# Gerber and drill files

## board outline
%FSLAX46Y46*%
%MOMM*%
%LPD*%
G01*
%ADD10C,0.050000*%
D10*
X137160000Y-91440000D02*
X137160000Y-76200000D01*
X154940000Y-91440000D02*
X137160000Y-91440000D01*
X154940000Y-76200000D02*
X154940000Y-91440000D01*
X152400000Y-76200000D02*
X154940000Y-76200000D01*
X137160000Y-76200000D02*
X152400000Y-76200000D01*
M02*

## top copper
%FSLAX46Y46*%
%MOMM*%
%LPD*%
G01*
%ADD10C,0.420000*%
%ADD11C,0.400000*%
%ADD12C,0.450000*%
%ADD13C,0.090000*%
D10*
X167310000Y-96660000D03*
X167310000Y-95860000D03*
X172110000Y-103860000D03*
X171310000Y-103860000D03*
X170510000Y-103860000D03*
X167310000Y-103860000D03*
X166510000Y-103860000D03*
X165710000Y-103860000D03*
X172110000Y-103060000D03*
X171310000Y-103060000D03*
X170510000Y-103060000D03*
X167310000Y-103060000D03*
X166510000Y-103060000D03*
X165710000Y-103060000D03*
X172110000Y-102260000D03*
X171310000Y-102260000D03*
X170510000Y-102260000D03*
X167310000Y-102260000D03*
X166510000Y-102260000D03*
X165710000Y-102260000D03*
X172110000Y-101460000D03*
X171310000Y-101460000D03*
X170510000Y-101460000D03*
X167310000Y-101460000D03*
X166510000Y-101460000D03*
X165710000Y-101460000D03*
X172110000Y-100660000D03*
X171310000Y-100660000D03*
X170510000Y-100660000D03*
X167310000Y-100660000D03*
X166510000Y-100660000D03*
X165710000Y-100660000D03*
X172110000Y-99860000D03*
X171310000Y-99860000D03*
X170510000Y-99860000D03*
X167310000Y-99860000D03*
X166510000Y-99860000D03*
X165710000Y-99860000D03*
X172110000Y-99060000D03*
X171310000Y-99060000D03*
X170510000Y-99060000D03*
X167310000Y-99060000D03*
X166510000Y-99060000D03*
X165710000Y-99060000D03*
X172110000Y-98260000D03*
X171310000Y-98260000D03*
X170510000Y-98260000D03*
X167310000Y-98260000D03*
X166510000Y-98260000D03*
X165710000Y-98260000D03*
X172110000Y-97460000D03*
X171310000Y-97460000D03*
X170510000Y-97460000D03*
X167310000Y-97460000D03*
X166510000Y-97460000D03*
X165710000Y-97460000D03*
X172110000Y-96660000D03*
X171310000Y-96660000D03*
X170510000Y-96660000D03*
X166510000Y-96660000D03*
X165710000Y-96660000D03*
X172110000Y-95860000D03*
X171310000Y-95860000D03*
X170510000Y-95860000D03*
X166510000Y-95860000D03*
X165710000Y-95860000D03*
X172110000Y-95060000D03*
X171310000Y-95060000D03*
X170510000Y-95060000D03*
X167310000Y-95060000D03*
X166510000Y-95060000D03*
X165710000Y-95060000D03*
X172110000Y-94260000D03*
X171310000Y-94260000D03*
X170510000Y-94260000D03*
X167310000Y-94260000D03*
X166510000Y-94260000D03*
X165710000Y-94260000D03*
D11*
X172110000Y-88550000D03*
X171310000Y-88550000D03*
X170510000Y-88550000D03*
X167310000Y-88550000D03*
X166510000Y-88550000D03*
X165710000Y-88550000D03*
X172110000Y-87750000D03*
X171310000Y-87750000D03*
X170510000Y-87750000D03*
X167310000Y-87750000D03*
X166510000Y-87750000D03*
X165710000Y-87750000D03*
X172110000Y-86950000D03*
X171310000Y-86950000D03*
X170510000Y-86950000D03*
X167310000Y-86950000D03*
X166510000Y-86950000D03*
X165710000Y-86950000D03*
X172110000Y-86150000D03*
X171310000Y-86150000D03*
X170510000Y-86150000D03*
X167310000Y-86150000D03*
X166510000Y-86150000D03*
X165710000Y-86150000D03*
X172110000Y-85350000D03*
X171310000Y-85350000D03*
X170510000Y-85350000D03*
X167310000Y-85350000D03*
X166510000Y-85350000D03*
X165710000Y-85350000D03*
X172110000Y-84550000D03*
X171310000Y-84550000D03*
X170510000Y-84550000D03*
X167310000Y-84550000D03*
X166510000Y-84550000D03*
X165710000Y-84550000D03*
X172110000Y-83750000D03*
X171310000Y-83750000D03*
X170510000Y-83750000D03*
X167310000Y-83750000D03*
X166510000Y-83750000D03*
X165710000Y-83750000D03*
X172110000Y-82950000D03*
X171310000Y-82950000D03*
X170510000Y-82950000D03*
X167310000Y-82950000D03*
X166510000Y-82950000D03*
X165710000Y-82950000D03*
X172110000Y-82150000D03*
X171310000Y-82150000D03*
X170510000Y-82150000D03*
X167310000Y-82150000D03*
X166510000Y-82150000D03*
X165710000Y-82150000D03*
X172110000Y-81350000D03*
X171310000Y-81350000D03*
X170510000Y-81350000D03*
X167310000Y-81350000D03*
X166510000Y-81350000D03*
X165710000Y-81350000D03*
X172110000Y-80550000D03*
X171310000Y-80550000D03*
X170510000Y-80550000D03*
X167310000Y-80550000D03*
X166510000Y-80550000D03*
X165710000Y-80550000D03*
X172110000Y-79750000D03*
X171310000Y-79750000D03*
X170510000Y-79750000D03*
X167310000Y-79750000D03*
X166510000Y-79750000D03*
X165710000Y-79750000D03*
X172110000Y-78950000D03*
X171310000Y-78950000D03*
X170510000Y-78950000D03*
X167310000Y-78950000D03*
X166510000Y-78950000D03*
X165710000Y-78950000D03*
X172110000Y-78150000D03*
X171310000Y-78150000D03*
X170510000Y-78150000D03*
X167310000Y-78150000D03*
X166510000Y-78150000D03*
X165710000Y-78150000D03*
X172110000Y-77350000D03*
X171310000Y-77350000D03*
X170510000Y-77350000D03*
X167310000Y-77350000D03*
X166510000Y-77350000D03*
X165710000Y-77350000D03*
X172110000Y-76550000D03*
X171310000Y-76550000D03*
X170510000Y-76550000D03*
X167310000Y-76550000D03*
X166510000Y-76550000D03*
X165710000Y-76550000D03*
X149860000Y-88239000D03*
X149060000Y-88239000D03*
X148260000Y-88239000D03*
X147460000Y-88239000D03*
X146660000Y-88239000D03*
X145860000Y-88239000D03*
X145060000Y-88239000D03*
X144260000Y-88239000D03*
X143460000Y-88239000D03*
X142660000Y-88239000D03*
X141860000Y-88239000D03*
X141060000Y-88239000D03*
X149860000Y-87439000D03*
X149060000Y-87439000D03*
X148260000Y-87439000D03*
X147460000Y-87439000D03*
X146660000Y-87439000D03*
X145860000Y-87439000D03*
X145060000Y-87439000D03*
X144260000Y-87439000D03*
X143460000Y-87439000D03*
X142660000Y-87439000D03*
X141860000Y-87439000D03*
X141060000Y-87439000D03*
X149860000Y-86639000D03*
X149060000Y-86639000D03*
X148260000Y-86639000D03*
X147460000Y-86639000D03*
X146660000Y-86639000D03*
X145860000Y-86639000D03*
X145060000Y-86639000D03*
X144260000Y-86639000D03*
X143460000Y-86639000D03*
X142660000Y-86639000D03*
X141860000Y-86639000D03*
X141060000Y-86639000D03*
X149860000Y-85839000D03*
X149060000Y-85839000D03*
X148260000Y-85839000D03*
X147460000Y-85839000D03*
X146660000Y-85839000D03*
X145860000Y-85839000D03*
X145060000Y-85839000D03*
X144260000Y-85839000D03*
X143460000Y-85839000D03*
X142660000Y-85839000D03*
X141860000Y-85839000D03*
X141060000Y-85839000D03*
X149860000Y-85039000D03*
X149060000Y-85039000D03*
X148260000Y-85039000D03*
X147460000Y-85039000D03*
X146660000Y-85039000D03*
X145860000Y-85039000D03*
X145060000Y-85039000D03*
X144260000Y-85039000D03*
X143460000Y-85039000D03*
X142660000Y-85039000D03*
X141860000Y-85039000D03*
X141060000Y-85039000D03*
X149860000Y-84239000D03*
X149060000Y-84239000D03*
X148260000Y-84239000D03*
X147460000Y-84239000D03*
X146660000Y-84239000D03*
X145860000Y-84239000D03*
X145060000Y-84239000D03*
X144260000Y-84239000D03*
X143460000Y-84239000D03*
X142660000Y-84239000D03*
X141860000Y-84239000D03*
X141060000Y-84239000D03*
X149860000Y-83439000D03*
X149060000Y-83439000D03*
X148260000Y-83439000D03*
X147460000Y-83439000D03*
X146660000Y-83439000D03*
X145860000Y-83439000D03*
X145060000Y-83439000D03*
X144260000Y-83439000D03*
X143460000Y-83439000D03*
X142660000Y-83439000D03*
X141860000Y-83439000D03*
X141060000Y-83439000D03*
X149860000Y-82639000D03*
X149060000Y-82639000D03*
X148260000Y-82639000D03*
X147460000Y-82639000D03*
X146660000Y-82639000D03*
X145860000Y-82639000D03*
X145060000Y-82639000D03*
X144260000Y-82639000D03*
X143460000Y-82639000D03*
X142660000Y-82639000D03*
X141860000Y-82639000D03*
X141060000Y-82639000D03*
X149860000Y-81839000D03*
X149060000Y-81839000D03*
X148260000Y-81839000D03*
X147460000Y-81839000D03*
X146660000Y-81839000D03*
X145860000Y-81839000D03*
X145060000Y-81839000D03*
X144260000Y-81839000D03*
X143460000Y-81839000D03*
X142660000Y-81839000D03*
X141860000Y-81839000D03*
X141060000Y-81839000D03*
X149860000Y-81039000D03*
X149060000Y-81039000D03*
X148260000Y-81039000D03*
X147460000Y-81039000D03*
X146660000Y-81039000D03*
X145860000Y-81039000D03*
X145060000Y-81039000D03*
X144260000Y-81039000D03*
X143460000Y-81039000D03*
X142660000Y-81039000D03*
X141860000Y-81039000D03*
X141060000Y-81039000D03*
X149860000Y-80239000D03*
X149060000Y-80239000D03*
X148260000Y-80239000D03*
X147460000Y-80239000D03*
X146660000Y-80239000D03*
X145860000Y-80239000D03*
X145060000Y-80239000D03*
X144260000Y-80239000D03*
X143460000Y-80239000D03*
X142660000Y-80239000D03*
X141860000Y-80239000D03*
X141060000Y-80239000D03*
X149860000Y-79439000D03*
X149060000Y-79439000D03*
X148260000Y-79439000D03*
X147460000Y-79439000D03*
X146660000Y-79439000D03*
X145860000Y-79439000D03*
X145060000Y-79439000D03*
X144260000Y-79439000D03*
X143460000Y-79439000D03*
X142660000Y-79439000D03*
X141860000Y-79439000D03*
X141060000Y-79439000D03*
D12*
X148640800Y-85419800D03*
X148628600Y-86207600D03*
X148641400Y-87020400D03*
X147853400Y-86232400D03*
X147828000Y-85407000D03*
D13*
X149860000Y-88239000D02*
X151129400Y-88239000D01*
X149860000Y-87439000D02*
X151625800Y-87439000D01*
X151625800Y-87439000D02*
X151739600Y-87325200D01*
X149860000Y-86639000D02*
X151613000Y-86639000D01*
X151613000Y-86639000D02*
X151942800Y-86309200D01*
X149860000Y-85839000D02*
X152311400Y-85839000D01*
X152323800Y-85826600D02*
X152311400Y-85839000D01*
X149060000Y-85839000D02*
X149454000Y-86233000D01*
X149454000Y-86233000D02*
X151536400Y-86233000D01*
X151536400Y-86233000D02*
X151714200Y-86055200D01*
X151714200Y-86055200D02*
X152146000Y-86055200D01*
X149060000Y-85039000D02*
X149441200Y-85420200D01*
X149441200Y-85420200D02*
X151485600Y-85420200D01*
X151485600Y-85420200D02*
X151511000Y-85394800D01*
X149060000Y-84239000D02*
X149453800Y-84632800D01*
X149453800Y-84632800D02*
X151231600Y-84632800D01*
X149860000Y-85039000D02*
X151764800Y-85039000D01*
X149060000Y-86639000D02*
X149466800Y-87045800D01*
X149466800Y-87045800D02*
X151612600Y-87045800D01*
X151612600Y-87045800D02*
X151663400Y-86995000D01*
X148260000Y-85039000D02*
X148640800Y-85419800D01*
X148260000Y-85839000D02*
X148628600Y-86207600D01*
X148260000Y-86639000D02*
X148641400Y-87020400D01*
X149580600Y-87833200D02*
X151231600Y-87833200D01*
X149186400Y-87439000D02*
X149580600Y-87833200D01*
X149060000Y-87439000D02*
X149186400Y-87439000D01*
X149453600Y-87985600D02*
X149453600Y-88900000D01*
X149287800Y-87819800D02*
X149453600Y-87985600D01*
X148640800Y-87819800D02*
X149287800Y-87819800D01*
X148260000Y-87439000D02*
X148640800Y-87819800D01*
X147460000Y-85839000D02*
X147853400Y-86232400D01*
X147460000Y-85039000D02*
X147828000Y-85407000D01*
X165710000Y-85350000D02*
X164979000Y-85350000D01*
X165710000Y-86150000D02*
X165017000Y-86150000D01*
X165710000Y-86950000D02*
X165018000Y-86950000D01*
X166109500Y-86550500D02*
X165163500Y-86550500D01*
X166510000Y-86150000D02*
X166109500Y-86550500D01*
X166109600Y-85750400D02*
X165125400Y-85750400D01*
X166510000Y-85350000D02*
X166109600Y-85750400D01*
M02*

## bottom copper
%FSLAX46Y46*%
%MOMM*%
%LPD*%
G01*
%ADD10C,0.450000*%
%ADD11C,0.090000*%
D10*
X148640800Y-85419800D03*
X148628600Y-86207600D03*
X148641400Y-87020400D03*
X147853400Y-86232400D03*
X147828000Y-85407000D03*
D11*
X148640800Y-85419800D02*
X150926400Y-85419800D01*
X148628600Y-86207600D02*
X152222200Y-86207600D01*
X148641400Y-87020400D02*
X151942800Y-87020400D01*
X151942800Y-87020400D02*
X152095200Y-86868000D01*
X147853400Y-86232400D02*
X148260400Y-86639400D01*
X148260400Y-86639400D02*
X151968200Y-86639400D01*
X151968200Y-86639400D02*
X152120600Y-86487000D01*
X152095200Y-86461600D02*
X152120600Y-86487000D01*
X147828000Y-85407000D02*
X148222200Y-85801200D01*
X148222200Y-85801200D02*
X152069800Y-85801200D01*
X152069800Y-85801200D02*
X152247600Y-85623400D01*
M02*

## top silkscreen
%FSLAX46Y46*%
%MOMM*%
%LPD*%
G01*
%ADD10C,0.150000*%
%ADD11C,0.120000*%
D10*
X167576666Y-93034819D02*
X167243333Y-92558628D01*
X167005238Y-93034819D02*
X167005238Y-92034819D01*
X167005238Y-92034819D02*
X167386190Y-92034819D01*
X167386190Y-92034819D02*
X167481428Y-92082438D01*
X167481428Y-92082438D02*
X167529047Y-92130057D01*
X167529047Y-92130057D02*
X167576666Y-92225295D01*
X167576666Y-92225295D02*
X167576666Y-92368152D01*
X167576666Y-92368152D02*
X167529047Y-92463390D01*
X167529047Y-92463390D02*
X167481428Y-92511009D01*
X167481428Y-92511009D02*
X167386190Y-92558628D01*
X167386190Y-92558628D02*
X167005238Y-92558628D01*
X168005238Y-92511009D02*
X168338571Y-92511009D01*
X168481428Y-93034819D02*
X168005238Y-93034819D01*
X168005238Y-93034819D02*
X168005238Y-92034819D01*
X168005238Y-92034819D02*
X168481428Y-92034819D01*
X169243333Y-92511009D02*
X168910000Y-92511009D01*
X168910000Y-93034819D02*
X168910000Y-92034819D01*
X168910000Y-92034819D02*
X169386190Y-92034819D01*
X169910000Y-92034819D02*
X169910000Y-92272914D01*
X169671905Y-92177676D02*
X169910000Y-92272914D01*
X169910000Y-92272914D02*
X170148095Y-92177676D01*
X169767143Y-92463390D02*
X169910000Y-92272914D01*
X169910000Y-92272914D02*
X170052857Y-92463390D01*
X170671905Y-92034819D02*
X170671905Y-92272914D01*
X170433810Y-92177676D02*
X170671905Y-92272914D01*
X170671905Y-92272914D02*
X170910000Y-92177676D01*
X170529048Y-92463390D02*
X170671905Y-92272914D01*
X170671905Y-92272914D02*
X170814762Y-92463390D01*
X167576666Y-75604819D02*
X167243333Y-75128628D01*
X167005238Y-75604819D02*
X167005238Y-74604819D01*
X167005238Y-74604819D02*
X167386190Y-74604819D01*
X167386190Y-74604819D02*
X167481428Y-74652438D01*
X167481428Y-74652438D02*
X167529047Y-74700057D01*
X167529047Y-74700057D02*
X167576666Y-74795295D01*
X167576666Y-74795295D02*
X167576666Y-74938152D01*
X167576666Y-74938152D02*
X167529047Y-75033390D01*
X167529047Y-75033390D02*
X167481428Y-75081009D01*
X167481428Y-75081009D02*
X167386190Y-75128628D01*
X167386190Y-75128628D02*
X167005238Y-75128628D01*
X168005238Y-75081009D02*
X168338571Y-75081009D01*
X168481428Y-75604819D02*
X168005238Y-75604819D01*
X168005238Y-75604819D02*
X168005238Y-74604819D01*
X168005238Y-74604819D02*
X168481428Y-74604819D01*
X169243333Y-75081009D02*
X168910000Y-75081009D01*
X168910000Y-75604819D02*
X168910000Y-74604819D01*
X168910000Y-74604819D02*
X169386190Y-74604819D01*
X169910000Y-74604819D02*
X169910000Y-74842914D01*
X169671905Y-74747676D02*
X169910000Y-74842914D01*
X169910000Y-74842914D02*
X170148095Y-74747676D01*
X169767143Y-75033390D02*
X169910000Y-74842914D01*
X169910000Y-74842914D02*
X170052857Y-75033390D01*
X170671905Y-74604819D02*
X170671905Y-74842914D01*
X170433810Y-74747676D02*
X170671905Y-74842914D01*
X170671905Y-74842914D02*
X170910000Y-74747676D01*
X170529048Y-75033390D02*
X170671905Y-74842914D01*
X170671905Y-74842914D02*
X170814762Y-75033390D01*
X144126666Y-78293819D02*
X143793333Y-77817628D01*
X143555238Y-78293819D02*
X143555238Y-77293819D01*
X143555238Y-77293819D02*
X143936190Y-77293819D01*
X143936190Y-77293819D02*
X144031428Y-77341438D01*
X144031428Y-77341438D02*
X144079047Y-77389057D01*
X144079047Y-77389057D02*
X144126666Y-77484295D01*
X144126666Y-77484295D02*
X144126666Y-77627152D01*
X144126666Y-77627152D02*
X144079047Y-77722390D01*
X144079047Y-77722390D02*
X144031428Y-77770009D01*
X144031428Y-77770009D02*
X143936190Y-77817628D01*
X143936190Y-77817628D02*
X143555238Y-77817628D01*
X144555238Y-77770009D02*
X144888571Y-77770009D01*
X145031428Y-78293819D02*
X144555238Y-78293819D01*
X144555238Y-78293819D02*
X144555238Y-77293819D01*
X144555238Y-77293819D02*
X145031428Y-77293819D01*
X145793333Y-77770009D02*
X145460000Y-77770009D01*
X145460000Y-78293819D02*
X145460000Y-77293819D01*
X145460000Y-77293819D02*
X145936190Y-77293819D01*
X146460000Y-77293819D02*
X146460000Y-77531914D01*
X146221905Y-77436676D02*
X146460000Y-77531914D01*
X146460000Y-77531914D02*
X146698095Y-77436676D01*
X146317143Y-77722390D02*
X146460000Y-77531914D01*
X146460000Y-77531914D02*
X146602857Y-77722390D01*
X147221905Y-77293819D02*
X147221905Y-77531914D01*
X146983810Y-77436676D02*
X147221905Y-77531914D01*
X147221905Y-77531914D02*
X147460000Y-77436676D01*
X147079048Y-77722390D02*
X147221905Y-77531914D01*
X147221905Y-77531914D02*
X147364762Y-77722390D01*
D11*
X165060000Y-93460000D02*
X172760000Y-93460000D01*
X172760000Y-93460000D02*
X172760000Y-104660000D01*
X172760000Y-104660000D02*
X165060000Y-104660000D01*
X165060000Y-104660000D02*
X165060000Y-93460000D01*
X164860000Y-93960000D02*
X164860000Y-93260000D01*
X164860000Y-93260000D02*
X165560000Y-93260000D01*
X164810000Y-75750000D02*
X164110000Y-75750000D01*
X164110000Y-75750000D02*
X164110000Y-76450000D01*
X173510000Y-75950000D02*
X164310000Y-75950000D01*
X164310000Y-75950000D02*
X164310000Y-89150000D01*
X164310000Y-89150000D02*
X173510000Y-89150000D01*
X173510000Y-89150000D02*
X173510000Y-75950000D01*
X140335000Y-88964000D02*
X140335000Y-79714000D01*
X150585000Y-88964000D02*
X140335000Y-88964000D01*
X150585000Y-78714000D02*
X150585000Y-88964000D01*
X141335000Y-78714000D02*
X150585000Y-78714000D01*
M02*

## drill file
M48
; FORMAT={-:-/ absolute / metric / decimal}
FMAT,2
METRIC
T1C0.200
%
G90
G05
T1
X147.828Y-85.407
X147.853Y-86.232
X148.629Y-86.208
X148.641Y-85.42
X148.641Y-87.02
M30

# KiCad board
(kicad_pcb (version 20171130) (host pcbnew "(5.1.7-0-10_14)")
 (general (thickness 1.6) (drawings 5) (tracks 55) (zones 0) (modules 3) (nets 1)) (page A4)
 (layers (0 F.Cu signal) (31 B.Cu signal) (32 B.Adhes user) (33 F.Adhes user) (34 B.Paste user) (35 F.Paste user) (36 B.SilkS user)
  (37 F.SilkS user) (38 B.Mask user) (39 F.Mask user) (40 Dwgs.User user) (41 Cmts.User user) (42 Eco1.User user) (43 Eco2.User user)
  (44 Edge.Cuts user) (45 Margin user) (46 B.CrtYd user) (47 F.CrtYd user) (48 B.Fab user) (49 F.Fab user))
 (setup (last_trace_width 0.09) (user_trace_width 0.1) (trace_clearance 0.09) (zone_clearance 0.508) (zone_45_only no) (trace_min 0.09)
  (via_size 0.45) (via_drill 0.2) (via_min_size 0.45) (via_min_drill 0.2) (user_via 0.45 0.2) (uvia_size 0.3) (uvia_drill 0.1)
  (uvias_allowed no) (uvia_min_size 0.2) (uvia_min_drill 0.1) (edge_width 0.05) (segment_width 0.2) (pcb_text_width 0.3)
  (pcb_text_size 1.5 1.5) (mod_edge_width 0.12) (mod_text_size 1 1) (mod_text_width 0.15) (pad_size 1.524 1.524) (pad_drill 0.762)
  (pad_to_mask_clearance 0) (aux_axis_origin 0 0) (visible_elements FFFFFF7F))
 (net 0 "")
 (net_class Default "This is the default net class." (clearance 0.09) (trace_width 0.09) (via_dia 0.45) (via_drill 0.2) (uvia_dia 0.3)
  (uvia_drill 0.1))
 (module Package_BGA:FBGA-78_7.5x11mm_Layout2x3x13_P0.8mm (layer F.Cu) (at 168.91 99.06)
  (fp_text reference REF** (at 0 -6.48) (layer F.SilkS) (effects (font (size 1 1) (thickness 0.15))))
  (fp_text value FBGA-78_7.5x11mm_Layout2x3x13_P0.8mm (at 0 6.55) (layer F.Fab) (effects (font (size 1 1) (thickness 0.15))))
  (fp_line (start -3.85 -5.6) (end 3.85 -5.6) (layer F.SilkS) (width 0.12))
  (fp_line (start 3.85 -5.6) (end 3.85 5.6) (layer F.SilkS) (width 0.12))
  (fp_line (start 3.85 5.6) (end -3.85 5.6) (layer F.SilkS) (width 0.12))
  (fp_line (start -3.85 5.6) (end -3.85 -5.6) (layer F.SilkS) (width 0.12))
  (fp_line (start -4.05 -5.1) (end -4.05 -5.8) (layer F.SilkS) (width 0.12))
  (fp_line (start -4.05 -5.8) (end -3.35 -5.8) (layer F.SilkS) (width 0.12))
  (pad D3 smd circle (at -1.6 -2.4) (size 0.42 0.42) (layers F.Cu F.Paste F.Mask))
  (pad C3 smd circle (at -1.6 -3.2) (size 0.42 0.42) (layers F.Cu F.Paste F.Mask))
  (pad N9 smd circle (at 3.2 4.8) (size 0.42 0.42) (layers F.Cu F.Paste F.Mask))
  (pad N8 smd circle (at 2.4 4.8) (size 0.42 0.42) (layers F.Cu F.Paste F.Mask))
  (pad N7 smd circle (at 1.6 4.8) (size 0.42 0.42) (layers F.Cu F.Paste F.Mask))
  (pad N3 smd circle (at -1.6 4.8) (size 0.42 0.42) (layers F.Cu F.Paste F.Mask))
  (pad N2 smd circle (at -2.4 4.8) (size 0.42 0.42) (layers F.Cu F.Paste F.Mask))
  (pad N1 smd circle (at -3.2 4.8) (size 0.42 0.42) (layers F.Cu F.Paste F.Mask))
  (pad M9 smd circle (at 3.2 4) (size 0.42 0.42) (layers F.Cu F.Paste F.Mask))
  (pad M8 smd circle (at 2.4 4) (size 0.42 0.42) (layers F.Cu F.Paste F.Mask))
  (pad M7 smd circle (at 1.6 4) (size 0.42 0.42) (layers F.Cu F.Paste F.Mask))
  (pad M3 smd circle (at -1.6 4) (size 0.42 0.42) (layers F.Cu F.Paste F.Mask))
  (pad M2 smd circle (at -2.4 4) (size 0.42 0.42) (layers F.Cu F.Paste F.Mask))
  (pad M1 smd circle (at -3.2 4) (size 0.42 0.42) (layers F.Cu F.Paste F.Mask))
  (pad L9 smd circle (at 3.2 3.2) (size 0.42 0.42) (layers F.Cu F.Paste F.Mask))
  (pad L8 smd circle (at 2.4 3.2) (size 0.42 0.42) (layers F.Cu F.Paste F.Mask))
  (pad L7 smd circle (at 1.6 3.2) (size 0.42 0.42) (layers F.Cu F.Paste F.Mask))
  (pad L3 smd circle (at -1.6 3.2) (size 0.42 0.42) (layers F.Cu F.Paste F.Mask))
  (pad L2 smd circle (at -2.4 3.2) (size 0.42 0.42) (layers F.Cu F.Paste F.Mask))
  (pad L1 smd circle (at -3.2 3.2) (size 0.42 0.42) (layers F.Cu F.Paste F.Mask))
  (pad K9 smd circle (at 3.2 2.4) (size 0.42 0.42) (layers F.Cu F.Paste F.Mask))
  (pad K8 smd circle (at 2.4 2.4) (size 0.42 0.42) (layers F.Cu F.Paste F.Mask))
  (pad K7 smd circle (at 1.6 2.4) (size 0.42 0.42) (layers F.Cu F.Paste F.Mask))
  (pad K3 smd circle (at -1.6 2.4) (size 0.42 0.42) (layers F.Cu F.Paste F.Mask))
  (pad K2 smd circle (at -2.4 2.4) (size 0.42 0.42) (layers F.Cu F.Paste F.Mask))
  (pad K1 smd circle (at -3.2 2.4) (size 0.42 0.42) (layers F.Cu F.Paste F.Mask))
  (pad J9 smd circle (at 3.2 1.6) (size 0.42 0.42) (layers F.Cu F.Paste F.Mask))
  (pad J8 smd circle (at 2.4 1.6) (size 0.42 0.42) (layers F.Cu F.Paste F.Mask))
  (pad J7 smd circle (at 1.6 1.6) (size 0.42 0.42) (layers F.Cu F.Paste F.Mask))
  (pad J3 smd circle (at -1.6 1.6) (size 0.42 0.42) (layers F.Cu F.Paste F.Mask))
  (pad J2 smd circle (at -2.4 1.6) (size 0.42 0.42) (layers F.Cu F.Paste F.Mask))
  (pad J1 smd circle (at -3.2 1.6) (size 0.42 0.42) (layers F.Cu F.Paste F.Mask))
  (pad H9 smd circle (at 3.2 0.8) (size 0.42 0.42) (layers F.Cu F.Paste F.Mask))
  (pad H8 smd circle (at 2.4 0.8) (size 0.42 0.42) (layers F.Cu F.Paste F.Mask))
  (pad H7 smd circle (at 1.6 0.8) (size 0.42 0.42) (layers F.Cu F.Paste F.Mask))
  (pad H3 smd circle (at -1.6 0.8) (size 0.42 0.42) (layers F.Cu F.Paste F.Mask))
  (pad H2 smd circle (at -2.4 0.8) (size 0.42 0.42) (layers F.Cu F.Paste F.Mask))
  (pad H1 smd circle (at -3.2 0.8) (size 0.42 0.42) (layers F.Cu F.Paste F.Mask))
  (pad G9 smd circle (at 3.2 0) (size 0.42 0.42) (layers F.Cu F.Paste F.Mask))
  (pad G8 smd circle (at 2.4 0) (size 0.42 0.42) (layers F.Cu F.Paste F.Mask))
  (pad G7 smd circle (at 1.6 0) (size 0.42 0.42) (layers F.Cu F.Paste F.Mask))
  (pad G3 smd circle (at -1.6 0) (size 0.42 0.42) (layers F.Cu F.Paste F.Mask))
  (pad G2 smd circle (at -2.4 0) (size 0.42 0.42) (layers F.Cu F.Paste F.Mask))
  (pad G1 smd circle (at -3.2 0) (size 0.42 0.42) (layers F.Cu F.Paste F.Mask))
  (pad F9 smd circle (at 3.2 -0.8) (size 0.42 0.42) (layers F.Cu F.Paste F.Mask))
  (pad F8 smd circle (at 2.4 -0.8) (size 0.42 0.42) (layers F.Cu F.Paste F.Mask))
  (pad F7 smd circle (at 1.6 -0.8) (size 0.42 0.42) (layers F.Cu F.Paste F.Mask))
  (pad F3 smd circle (at -1.6 -0.8) (size 0.42 0.42) (layers F.Cu F.Paste F.Mask))
  (pad F2 smd circle (at -2.4 -0.8) (size 0.42 0.42) (layers F.Cu F.Paste F.Mask))
  (pad F1 smd circle (at -3.2 -0.8) (size 0.42 0.42) (layers F.Cu F.Paste F.Mask))
  (pad E9 smd circle (at 3.2 -1.6) (size 0.42 0.42) (layers F.Cu F.Paste F.Mask))
  (pad E8 smd circle (at 2.4 -1.6) (size 0.42 0.42) (layers F.Cu F.Paste F.Mask))
  (pad E7 smd circle (at 1.6 -1.6) (size 0.42 0.42) (layers F.Cu F.Paste F.Mask))
  (pad E3 smd circle (at -1.6 -1.6) (size 0.42 0.42) (layers F.Cu F.Paste F.Mask))
  (pad E2 smd circle (at -2.4 -1.6) (size 0.42 0.42) (layers F.Cu F.Paste F.Mask))
  (pad E1 smd circle (at -3.2 -1.6) (size 0.42 0.42) (layers F.Cu F.Paste F.Mask))
  (pad D9 smd circle (at 3.2 -2.4) (size 0.42 0.42) (layers F.Cu F.Paste F.Mask))
  (pad D8 smd circle (at 2.4 -2.4) (size 0.42 0.42) (layers F.Cu F.Paste F.Mask))
  (pad D7 smd circle (at 1.6 -2.4) (size 0.42 0.42) (layers F.Cu F.Paste F.Mask))
  (pad D2 smd circle (at -2.4 -2.4) (size 0.42 0.42) (layers F.Cu F.Paste F.Mask))
  (pad D1 smd circle (at -3.2 -2.4) (size 0.42 0.42) (layers F.Cu F.Paste F.Mask))
  (pad C9 smd circle (at 3.2 -3.2) (size 0.42 0.42) (layers F.Cu F.Paste F.Mask))
  (pad C8 smd circle (at 2.4 -3.2) (size 0.42 0.42) (layers F.Cu F.Paste F.Mask))
  (pad C7 smd circle (at 1.6 -3.2) (size 0.42 0.42) (layers F.Cu F.Paste F.Mask))
  (pad C2 smd circle (at -2.4 -3.2) (size 0.42 0.42) (layers F.Cu F.Paste F.Mask))
  (pad C1 smd circle (at -3.2 -3.2) (size 0.42 0.42) (layers F.Cu F.Paste F.Mask))
  (pad B9 smd circle (at 3.2 -4) (size 0.42 0.42) (layers F.Cu F.Paste F.Mask))
  (pad B8 smd circle (at 2.4 -4) (size 0.42 0.42) (layers F.Cu F.Paste F.Mask))
  (pad B7 smd circle (at 1.6 -4) (size 0.42 0.42) (layers F.Cu F.Paste F.Mask))
  (pad B3 smd circle (at -1.6 -4) (size 0.42 0.42) (layers F.Cu F.Paste F.Mask))
  (pad B2 smd circle (at -2.4 -4) (size 0.42 0.42) (layers F.Cu F.Paste F.Mask))
  (pad B1 smd circle (at -3.2 -4) (size 0.42 0.42) (layers F.Cu F.Paste F.Mask))
  (pad A9 smd circle (at 3.2 -4.8) (size 0.42 0.42) (layers F.Cu F.Paste F.Mask))
  (pad A8 smd circle (at 2.4 -4.8) (size 0.42 0.42) (layers F.Cu F.Paste F.Mask))
  (pad A7 smd circle (at 1.6 -4.8) (size 0.42 0.42) (layers F.Cu F.Paste F.Mask))
  (pad A3 smd circle (at -1.6 -4.8) (size 0.42 0.42) (layers F.Cu F.Paste F.Mask))
  (pad A2 smd circle (at -2.4 -4.8) (size 0.42 0.42) (layers F.Cu F.Paste F.Mask))
  (pad A1 smd circle (at -3.2 -4.8) (size 0.42 0.42) (layers F.Cu F.Paste F.Mask)))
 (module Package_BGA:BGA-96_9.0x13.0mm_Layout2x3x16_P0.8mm (layer F.Cu) (at 168.91 82.55)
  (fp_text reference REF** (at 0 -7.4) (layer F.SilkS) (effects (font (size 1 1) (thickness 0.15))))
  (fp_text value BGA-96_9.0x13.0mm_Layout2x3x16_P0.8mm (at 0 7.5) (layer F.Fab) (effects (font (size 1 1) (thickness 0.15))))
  (fp_line (start -4.1 -6.8) (end -4.8 -6.8) (layer F.SilkS) (width 0.12))
  (fp_line (start -4.8 -6.8) (end -4.8 -6.1) (layer F.SilkS) (width 0.12))
  (fp_line (start 4.6 -6.6) (end -4.6 -6.6) (layer F.SilkS) (width 0.12))
  (fp_line (start -4.6 -6.6) (end -4.6 6.6) (layer F.SilkS) (width 0.12))
  (fp_line (start -4.6 6.6) (end 4.6 6.6) (layer F.SilkS) (width 0.12))
  (fp_line (start 4.6 6.6) (end 4.6 -6.6) (layer F.SilkS) (width 0.12))
  (pad T9 smd circle (at 3.2 6) (size 0.4 0.4) (layers F.Cu F.Paste F.Mask))
  (pad T8 smd circle (at 2.4 6) (size 0.4 0.4) (layers F.Cu F.Paste F.Mask))
  (pad T7 smd circle (at 1.6 6) (size 0.4 0.4) (layers F.Cu F.Paste F.Mask))
  (pad T3 smd circle (at -1.6 6) (size 0.4 0.4) (layers F.Cu F.Paste F.Mask))
  (pad T2 smd circle (at -2.4 6) (size 0.4 0.4) (layers F.Cu F.Paste F.Mask))
  (pad T1 smd circle (at -3.2 6) (size 0.4 0.4) (layers F.Cu F.Paste F.Mask))
  (pad R9 smd circle (at 3.2 5.2) (size 0.4 0.4) (layers F.Cu F.Paste F.Mask))
  (pad R8 smd circle (at 2.4 5.2) (size 0.4 0.4) (layers F.Cu F.Paste F.Mask))
  (pad R7 smd circle (at 1.6 5.2) (size 0.4 0.4) (layers F.Cu F.Paste F.Mask))
  (pad R3 smd circle (at -1.6 5.2) (size 0.4 0.4) (layers F.Cu F.Paste F.Mask))
  (pad R2 smd circle (at -2.4 5.2) (size 0.4 0.4) (layers F.Cu F.Paste F.Mask))
  (pad R1 smd circle (at -3.2 5.2) (size 0.4 0.4) (layers F.Cu F.Paste F.Mask))
  (pad P9 smd circle (at 3.2 4.4) (size 0.4 0.4) (layers F.Cu F.Paste F.Mask))
  (pad P8 smd circle (at 2.4 4.4) (size 0.4 0.4) (layers F.Cu F.Paste F.Mask))
  (pad P7 smd circle (at 1.6 4.4) (size 0.4 0.4) (layers F.Cu F.Paste F.Mask))
  (pad P3 smd circle (at -1.6 4.4) (size 0.4 0.4) (layers F.Cu F.Paste F.Mask))
  (pad P2 smd circle (at -2.4 4.4) (size 0.4 0.4) (layers F.Cu F.Paste F.Mask))
  (pad P1 smd circle (at -3.2 4.4) (size 0.4 0.4) (layers F.Cu F.Paste F.Mask))
  (pad N9 smd circle (at 3.2 3.6) (size 0.4 0.4) (layers F.Cu F.Paste F.Mask))
  (pad N8 smd circle (at 2.4 3.6) (size 0.4 0.4) (layers F.Cu F.Paste F.Mask))
  (pad N7 smd circle (at 1.6 3.6) (size 0.4 0.4) (layers F.Cu F.Paste F.Mask))
  (pad N3 smd circle (at -1.6 3.6) (size 0.4 0.4) (layers F.Cu F.Paste F.Mask))
  (pad N2 smd circle (at -2.4 3.6) (size 0.4 0.4) (layers F.Cu F.Paste F.Mask))
  (pad N1 smd circle (at -3.2 3.6) (size 0.4 0.4) (layers F.Cu F.Paste F.Mask))
  (pad M9 smd circle (at 3.2 2.8) (size 0.4 0.4) (layers F.Cu F.Paste F.Mask))
  (pad M8 smd circle (at 2.4 2.8) (size 0.4 0.4) (layers F.Cu F.Paste F.Mask))
  (pad M7 smd circle (at 1.6 2.8) (size 0.4 0.4) (layers F.Cu F.Paste F.Mask))
  (pad M3 smd circle (at -1.6 2.8) (size 0.4 0.4) (layers F.Cu F.Paste F.Mask))
  (pad M2 smd circle (at -2.4 2.8) (size 0.4 0.4) (layers F.Cu F.Paste F.Mask))
  (pad M1 smd circle (at -3.2 2.8) (size 0.4 0.4) (layers F.Cu F.Paste F.Mask))
  (pad L9 smd circle (at 3.2 2) (size 0.4 0.4) (layers F.Cu F.Paste F.Mask))
  (pad L8 smd circle (at 2.4 2) (size 0.4 0.4) (layers F.Cu F.Paste F.Mask))
  (pad L7 smd circle (at 1.6 2) (size 0.4 0.4) (layers F.Cu F.Paste F.Mask))
  (pad L3 smd circle (at -1.6 2) (size 0.4 0.4) (layers F.Cu F.Paste F.Mask))
  (pad L2 smd circle (at -2.4 2) (size 0.4 0.4) (layers F.Cu F.Paste F.Mask))
  (pad L1 smd circle (at -3.2 2) (size 0.4 0.4) (layers F.Cu F.Paste F.Mask))
  (pad K9 smd circle (at 3.2 1.2) (size 0.4 0.4) (layers F.Cu F.Paste F.Mask))
  (pad K8 smd circle (at 2.4 1.2) (size 0.4 0.4) (layers F.Cu F.Paste F.Mask))
  (pad K7 smd circle (at 1.6 1.2) (size 0.4 0.4) (layers F.Cu F.Paste F.Mask))
  (pad K3 smd circle (at -1.6 1.2) (size 0.4 0.4) (layers F.Cu F.Paste F.Mask))
  (pad K2 smd circle (at -2.4 1.2) (size 0.4 0.4) (layers F.Cu F.Paste F.Mask))
  (pad K1 smd circle (at -3.2 1.2) (size 0.4 0.4) (layers F.Cu F.Paste F.Mask))
  (pad J9 smd circle (at 3.2 0.4) (size 0.4 0.4) (layers F.Cu F.Paste F.Mask))
  (pad J8 smd circle (at 2.4 0.4) (size 0.4 0.4) (layers F.Cu F.Paste F.Mask))
  (pad J7 smd circle (at 1.6 0.4) (size 0.4 0.4) (layers F.Cu F.Paste F.Mask))
  (pad J3 smd circle (at -1.6 0.4) (size 0.4 0.4) (layers F.Cu F.Paste F.Mask))
  (pad J2 smd circle (at -2.4 0.4) (size 0.4 0.4) (layers F.Cu F.Paste F.Mask))
  (pad J1 smd circle (at -3.2 0.4) (size 0.4 0.4) (layers F.Cu F.Paste F.Mask))
  (pad H9 smd circle (at 3.2 -0.4) (size 0.4 0.4) (layers F.Cu F.Paste F.Mask))
  (pad H8 smd circle (at 2.4 -0.4) (size 0.4 0.4) (layers F.Cu F.Paste F.Mask))
  (pad H7 smd circle (at 1.6 -0.4) (size 0.4 0.4) (layers F.Cu F.Paste F.Mask))
  (pad H3 smd circle (at -1.6 -0.4) (size 0.4 0.4) (layers F.Cu F.Paste F.Mask))
  (pad H2 smd circle (at -2.4 -0.4) (size 0.4 0.4) (layers F.Cu F.Paste F.Mask))
  (pad H1 smd circle (at -3.2 -0.4) (size 0.4 0.4) (layers F.Cu F.Paste F.Mask))
  (pad G9 smd circle (at 3.2 -1.2) (size 0.4 0.4) (layers F.Cu F.Paste F.Mask))
  (pad G8 smd circle (at 2.4 -1.2) (size 0.4 0.4) (layers F.Cu F.Paste F.Mask))
  (pad G7 smd circle (at 1.6 -1.2) (size 0.4 0.4) (layers F.Cu F.Paste F.Mask))
  (pad G3 smd circle (at -1.6 -1.2) (size 0.4 0.4) (layers F.Cu F.Paste F.Mask))
  (pad G2 smd circle (at -2.4 -1.2) (size 0.4 0.4) (layers F.Cu F.Paste F.Mask))
  (pad G1 smd circle (at -3.2 -1.2) (size 0.4 0.4) (layers F.Cu F.Paste F.Mask))
  (pad F9 smd circle (at 3.2 -2) (size 0.4 0.4) (layers F.Cu F.Paste F.Mask))
  (pad F8 smd circle (at 2.4 -2) (size 0.4 0.4) (layers F.Cu F.Paste F.Mask))
  (pad F7 smd circle (at 1.6 -2) (size 0.4 0.4) (layers F.Cu F.Paste F.Mask))
  (pad F3 smd circle (at -1.6 -2) (size 0.4 0.4) (layers F.Cu F.Paste F.Mask))
  (pad F2 smd circle (at -2.4 -2) (size 0.4 0.4) (layers F.Cu F.Paste F.Mask))
  (pad F1 smd circle (at -3.2 -2) (size 0.4 0.4) (layers F.Cu F.Paste F.Mask))
  (pad E9 smd circle (at 3.2 -2.8) (size 0.4 0.4) (layers F.Cu F.Paste F.Mask))
  (pad E8 smd circle (at 2.4 -2.8) (size 0.4 0.4) (layers F.Cu F.Paste F.Mask))
  (pad E7 smd circle (at 1.6 -2.8) (size 0.4 0.4) (layers F.Cu F.Paste F.Mask))
  (pad E3 smd circle (at -1.6 -2.8) (size 0.4 0.4) (layers F.Cu F.Paste F.Mask))
  (pad E2 smd circle (at -2.4 -2.8) (size 0.4 0.4) (layers F.Cu F.Paste F.Mask))
  (pad E1 smd circle (at -3.2 -2.8) (size 0.4 0.4) (layers F.Cu F.Paste F.Mask))
  (pad D9 smd circle (at 3.2 -3.6) (size 0.4 0.4) (layers F.Cu F.Paste F.Mask))
  (pad D8 smd circle (at 2.4 -3.6) (size 0.4 0.4) (layers F.Cu F.Paste F.Mask))
  (pad D7 smd circle (at 1.6 -3.6) (size 0.4 0.4) (layers F.Cu F.Paste F.Mask))
  (pad D3 smd circle (at -1.6 -3.6) (size 0.4 0.4) (layers F.Cu F.Paste F.Mask))
  (pad D2 smd circle (at -2.4 -3.6) (size 0.4 0.4) (layers F.Cu F.Paste F.Mask))
  (pad D1 smd circle (at -3.2 -3.6) (size 0.4 0.4) (layers F.Cu F.Paste F.Mask))
  (pad C9 smd circle (at 3.2 -4.4) (size 0.4 0.4) (layers F.Cu F.Paste F.Mask))
  (pad C8 smd circle (at 2.4 -4.4) (size 0.4 0.4) (layers F.Cu F.Paste F.Mask))
  (pad C7 smd circle (at 1.6 -4.4) (size 0.4 0.4) (layers F.Cu F.Paste F.Mask))
  (pad C3 smd circle (at -1.6 -4.4) (size 0.4 0.4) (layers F.Cu F.Paste F.Mask))
  (pad C2 smd circle (at -2.4 -4.4) (size 0.4 0.4) (layers F.Cu F.Paste F.Mask))
  (pad C1 smd circle (at -3.2 -4.4) (size 0.4 0.4) (layers F.Cu F.Paste F.Mask))
  (pad B9 smd circle (at 3.2 -5.2) (size 0.4 0.4) (layers F.Cu F.Paste F.Mask))
  (pad B8 smd circle (at 2.4 -5.2) (size 0.4 0.4) (layers F.Cu F.Paste F.Mask))
  (pad B7 smd circle (at 1.6 -5.2) (size 0.4 0.4) (layers F.Cu F.Paste F.Mask))
  (pad B3 smd circle (at -1.6 -5.2) (size 0.4 0.4) (layers F.Cu F.Paste F.Mask))
  (pad B2 smd circle (at -2.4 -5.2) (size 0.4 0.4) (layers F.Cu F.Paste F.Mask))
  (pad B1 smd circle (at -3.2 -5.2) (size 0.4 0.4) (layers F.Cu F.Paste F.Mask))
  (pad A9 smd circle (at 3.2 -6) (size 0.4 0.4) (layers F.Cu F.Paste F.Mask))
  (pad A8 smd circle (at 2.4 -6) (size 0.4 0.4) (layers F.Cu F.Paste F.Mask))
  (pad A7 smd circle (at 1.6 -6) (size 0.4 0.4) (layers F.Cu F.Paste F.Mask))
  (pad A3 smd circle (at -1.6 -6) (size 0.4 0.4) (layers F.Cu F.Paste F.Mask))
  (pad A2 smd circle (at -2.4 -6) (size 0.4 0.4) (layers F.Cu F.Paste F.Mask))
  (pad A1 smd circle (at -3.2 -6) (size 0.4 0.4) (layers F.Cu F.Paste F.Mask)))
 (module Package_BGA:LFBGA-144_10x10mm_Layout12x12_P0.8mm (layer F.Cu) (at 145.46 83.839)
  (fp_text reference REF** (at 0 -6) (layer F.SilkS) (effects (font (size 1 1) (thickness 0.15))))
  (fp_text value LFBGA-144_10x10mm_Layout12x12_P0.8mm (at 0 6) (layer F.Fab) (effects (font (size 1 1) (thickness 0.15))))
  (fp_line (start -5.125 5.125) (end -5.125 -4.125) (layer F.SilkS) (width 0.12))
  (fp_line (start 5.125 5.125) (end -5.125 5.125) (layer F.SilkS) (width 0.12))
  (fp_line (start 5.125 -5.125) (end 5.125 5.125) (layer F.SilkS) (width 0.12))
  (fp_line (start -4.125 -5.125) (end 5.125 -5.125) (layer F.SilkS) (width 0.12))
  (pad M12 smd circle (at 4.4 4.4) (size 0.4 0.4) (layers F.Cu F.Paste F.Mask))
  (pad M11 smd circle (at 3.6 4.4) (size 0.4 0.4) (layers F.Cu F.Paste F.Mask))
  (pad M10 smd circle (at 2.8 4.4) (size 0.4 0.4) (layers F.Cu F.Paste F.Mask))
  (pad M9 smd circle (at 2 4.4) (size 0.4 0.4) (layers F.Cu F.Paste F.Mask))
  (pad M8 smd circle (at 1.2 4.4) (size 0.4 0.4) (layers F.Cu F.Paste F.Mask))
  (pad M7 smd circle (at 0.4 4.4) (size 0.4 0.4) (layers F.Cu F.Paste F.Mask))
  (pad M6 smd circle (at -0.4 4.4) (size 0.4 0.4) (layers F.Cu F.Paste F.Mask))
  (pad M5 smd circle (at -1.2 4.4) (size 0.4 0.4) (layers F.Cu F.Paste F.Mask))
  (pad M4 smd circle (at -2 4.4) (size 0.4 0.4) (layers F.Cu F.Paste F.Mask))
  (pad M3 smd circle (at -2.8 4.4) (size 0.4 0.4) (layers F.Cu F.Paste F.Mask))
  (pad M2 smd circle (at -3.6 4.4) (size 0.4 0.4) (layers F.Cu F.Paste F.Mask))
  (pad M1 smd circle (at -4.4 4.4) (size 0.4 0.4) (layers F.Cu F.Paste F.Mask))
  (pad L12 smd circle (at 4.4 3.6) (size 0.4 0.4) (layers F.Cu F.Paste F.Mask))
  (pad L11 smd circle (at 3.6 3.6) (size 0.4 0.4) (layers F.Cu F.Paste F.Mask))
  (pad L10 smd circle (at 2.8 3.6) (size 0.4 0.4) (layers F.Cu F.Paste F.Mask))
  (pad L9 smd circle (at 2 3.6) (size 0.4 0.4) (layers F.Cu F.Paste F.Mask))
  (pad L8 smd circle (at 1.2 3.6) (size 0.4 0.4) (layers F.Cu F.Paste F.Mask))
  (pad L7 smd circle (at 0.4 3.6) (size 0.4 0.4) (layers F.Cu F.Paste F.Mask))
  (pad L6 smd circle (at -0.4 3.6) (size 0.4 0.4) (layers F.Cu F.Paste F.Mask))
  (pad L5 smd circle (at -1.2 3.6) (size 0.4 0.4) (layers F.Cu F.Paste F.Mask))
  (pad L4 smd circle (at -2 3.6) (size 0.4 0.4) (layers F.Cu F.Paste F.Mask))
  (pad L3 smd circle (at -2.8 3.6) (size 0.4 0.4) (layers F.Cu F.Paste F.Mask))
  (pad L2 smd circle (at -3.6 3.6) (size 0.4 0.4) (layers F.Cu F.Paste F.Mask))
  (pad L1 smd circle (at -4.4 3.6) (size 0.4 0.4) (layers F.Cu F.Paste F.Mask))
  (pad K12 smd circle (at 4.4 2.8) (size 0.4 0.4) (layers F.Cu F.Paste F.Mask))
  (pad K11 smd circle (at 3.6 2.8) (size 0.4 0.4) (layers F.Cu F.Paste F.Mask))
  (pad K10 smd circle (at 2.8 2.8) (size 0.4 0.4) (layers F.Cu F.Paste F.Mask))
  (pad K9 smd circle (at 2 2.8) (size 0.4 0.4) (layers F.Cu F.Paste F.Mask))
  (pad K8 smd circle (at 1.2 2.8) (size 0.4 0.4) (layers F.Cu F.Paste F.Mask))
  (pad K7 smd circle (at 0.4 2.8) (size 0.4 0.4) (layers F.Cu F.Paste F.Mask))
  (pad K6 smd circle (at -0.4 2.8) (size 0.4 0.4) (layers F.Cu F.Paste F.Mask))
  (pad K5 smd circle (at -1.2 2.8) (size 0.4 0.4) (layers F.Cu F.Paste F.Mask))
  (pad K4 smd circle (at -2 2.8) (size 0.4 0.4) (layers F.Cu F.Paste F.Mask))
  (pad K3 smd circle (at -2.8 2.8) (size 0.4 0.4) (layers F.Cu F.Paste F.Mask))
  (pad K2 smd circle (at -3.6 2.8) (size 0.4 0.4) (layers F.Cu F.Paste F.Mask))
  (pad K1 smd circle (at -4.4 2.8) (size 0.4 0.4) (layers F.Cu F.Paste F.Mask))
  (pad J12 smd circle (at 4.4 2) (size 0.4 0.4) (layers F.Cu F.Paste F.Mask))
  (pad J11 smd circle (at 3.6 2) (size 0.4 0.4) (layers F.Cu F.Paste F.Mask))
  (pad J10 smd circle (at 2.8 2) (size 0.4 0.4) (layers F.Cu F.Paste F.Mask))
  (pad J9 smd circle (at 2 2) (size 0.4 0.4) (layers F.Cu F.Paste F.Mask))
  (pad J8 smd circle (at 1.2 2) (size 0.4 0.4) (layers F.Cu F.Paste F.Mask))
  (pad J7 smd circle (at 0.4 2) (size 0.4 0.4) (layers F.Cu F.Paste F.Mask))
  (pad J6 smd circle (at -0.4 2) (size 0.4 0.4) (layers F.Cu F.Paste F.Mask))
  (pad J5 smd circle (at -1.2 2) (size 0.4 0.4) (layers F.Cu F.Paste F.Mask))
  (pad J4 smd circle (at -2 2) (size 0.4 0.4) (layers F.Cu F.Paste F.Mask))
  (pad J3 smd circle (at -2.8 2) (size 0.4 0.4) (layers F.Cu F.Paste F.Mask))
  (pad J2 smd circle (at -3.6 2) (size 0.4 0.4) (layers F.Cu F.Paste F.Mask))
  (pad J1 smd circle (at -4.4 2) (size 0.4 0.4) (layers F.Cu F.Paste F.Mask))
  (pad H12 smd circle (at 4.4 1.2) (size 0.4 0.4) (layers F.Cu F.Paste F.Mask))
  (pad H11 smd circle (at 3.6 1.2) (size 0.4 0.4) (layers F.Cu F.Paste F.Mask))
  (pad H10 smd circle (at 2.8 1.2) (size 0.4 0.4) (layers F.Cu F.Paste F.Mask))
  (pad H9 smd circle (at 2 1.2) (size 0.4 0.4) (layers F.Cu F.Paste F.Mask))
  (pad H8 smd circle (at 1.2 1.2) (size 0.4 0.4) (layers F.Cu F.Paste F.Mask))
  (pad H7 smd circle (at 0.4 1.2) (size 0.4 0.4) (layers F.Cu F.Paste F.Mask))
  (pad H6 smd circle (at -0.4 1.2) (size 0.4 0.4) (layers F.Cu F.Paste F.Mask))
  (pad H5 smd circle (at -1.2 1.2) (size 0.4 0.4) (layers F.Cu F.Paste F.Mask))
  (pad H4 smd circle (at -2 1.2) (size 0.4 0.4) (layers F.Cu F.Paste F.Mask))
  (pad H3 smd circle (at -2.8 1.2) (size 0.4 0.4) (layers F.Cu F.Paste F.Mask))
  (pad H2 smd circle (at -3.6 1.2) (size 0.4 0.4) (layers F.Cu F.Paste F.Mask))
  (pad H1 smd circle (at -4.4 1.2) (size 0.4 0.4) (layers F.Cu F.Paste F.Mask))
  (pad G12 smd circle (at 4.4 0.4) (size 0.4 0.4) (layers F.Cu F.Paste F.Mask))
  (pad G11 smd circle (at 3.6 0.4) (size 0.4 0.4) (layers F.Cu F.Paste F.Mask))
  (pad G10 smd circle (at 2.8 0.4) (size 0.4 0.4) (layers F.Cu F.Paste F.Mask))
  (pad G9 smd circle (at 2 0.4) (size 0.4 0.4) (layers F.Cu F.Paste F.Mask))
  (pad G8 smd circle (at 1.2 0.4) (size 0.4 0.4) (layers F.Cu F.Paste F.Mask))
  (pad G7 smd circle (at 0.4 0.4) (size 0.4 0.4) (layers F.Cu F.Paste F.Mask))
  (pad G6 smd circle (at -0.4 0.4) (size 0.4 0.4) (layers F.Cu F.Paste F.Mask))
  (pad G5 smd circle (at -1.2 0.4) (size 0.4 0.4) (layers F.Cu F.Paste F.Mask))
  (pad G4 smd circle (at -2 0.4) (size 0.4 0.4) (layers F.Cu F.Paste F.Mask))
  (pad G3 smd circle (at -2.8 0.4) (size 0.4 0.4) (layers F.Cu F.Paste F.Mask))
  (pad G2 smd circle (at -3.6 0.4) (size 0.4 0.4) (layers F.Cu F.Paste F.Mask))
  (pad G1 smd circle (at -4.4 0.4) (size 0.4 0.4) (layers F.Cu F.Paste F.Mask))
  (pad F12 smd circle (at 4.4 -0.4) (size 0.4 0.4) (layers F.Cu F.Paste F.Mask))
  (pad F11 smd circle (at 3.6 -0.4) (size 0.4 0.4) (layers F.Cu F.Paste F.Mask))
  (pad F10 smd circle (at 2.8 -0.4) (size 0.4 0.4) (layers F.Cu F.Paste F.Mask))
  (pad F9 smd circle (at 2 -0.4) (size 0.4 0.4) (layers F.Cu F.Paste F.Mask))
  (pad F8 smd circle (at 1.2 -0.4) (size 0.4 0.4) (layers F.Cu F.Paste F.Mask))
  (pad F7 smd circle (at 0.4 -0.4) (size 0.4 0.4) (layers F.Cu F.Paste F.Mask))
  (pad F6 smd circle (at -0.4 -0.4) (size 0.4 0.4) (layers F.Cu F.Paste F.Mask))
  (pad F5 smd circle (at -1.2 -0.4) (size 0.4 0.4) (layers F.Cu F.Paste F.Mask))
  (pad F4 smd circle (at -2 -0.4) (size 0.4 0.4) (layers F.Cu F.Paste F.Mask))
  (pad F3 smd circle (at -2.8 -0.4) (size 0.4 0.4) (layers F.Cu F.Paste F.Mask))
  (pad F2 smd circle (at -3.6 -0.4) (size 0.4 0.4) (layers F.Cu F.Paste F.Mask))
  (pad F1 smd circle (at -4.4 -0.4) (size 0.4 0.4) (layers F.Cu F.Paste F.Mask))
  (pad E12 smd circle (at 4.4 -1.2) (size 0.4 0.4) (layers F.Cu F.Paste F.Mask))
  (pad E11 smd circle (at 3.6 -1.2) (size 0.4 0.4) (layers F.Cu F.Paste F.Mask))
  (pad E10 smd circle (at 2.8 -1.2) (size 0.4 0.4) (layers F.Cu F.Paste F.Mask))
  (pad E9 smd circle (at 2 -1.2) (size 0.4 0.4) (layers F.Cu F.Paste F.Mask))
  (pad E8 smd circle (at 1.2 -1.2) (size 0.4 0.4) (layers F.Cu F.Paste F.Mask))
  (pad E7 smd circle (at 0.4 -1.2) (size 0.4 0.4) (layers F.Cu F.Paste F.Mask))
  (pad E6 smd circle (at -0.4 -1.2) (size 0.4 0.4) (layers F.Cu F.Paste F.Mask))
  (pad E5 smd circle (at -1.2 -1.2) (size 0.4 0.4) (layers F.Cu F.Paste F.Mask))
  (pad E4 smd circle (at -2 -1.2) (size 0.4 0.4) (layers F.Cu F.Paste F.Mask))
  (pad E3 smd circle (at -2.8 -1.2) (size 0.4 0.4) (layers F.Cu F.Paste F.Mask))
  (pad E2 smd circle (at -3.6 -1.2) (size 0.4 0.4) (layers F.Cu F.Paste F.Mask))
  (pad E1 smd circle (at -4.4 -1.2) (size 0.4 0.4) (layers F.Cu F.Paste F.Mask))
  (pad D12 smd circle (at 4.4 -2) (size 0.4 0.4) (layers F.Cu F.Paste F.Mask))
  (pad D11 smd circle (at 3.6 -2) (size 0.4 0.4) (layers F.Cu F.Paste F.Mask))
  (pad D10 smd circle (at 2.8 -2) (size 0.4 0.4) (layers F.Cu F.Paste F.Mask))
  (pad D9 smd circle (at 2 -2) (size 0.4 0.4) (layers F.Cu F.Paste F.Mask))
  (pad D8 smd circle (at 1.2 -2) (size 0.4 0.4) (layers F.Cu F.Paste F.Mask))
  (pad D7 smd circle (at 0.4 -2) (size 0.4 0.4) (layers F.Cu F.Paste F.Mask))
  (pad D6 smd circle (at -0.4 -2) (size 0.4 0.4) (layers F.Cu F.Paste F.Mask))
  (pad D5 smd circle (at -1.2 -2) (size 0.4 0.4) (layers F.Cu F.Paste F.Mask))
  (pad D4 smd circle (at -2 -2) (size 0.4 0.4) (layers F.Cu F.Paste F.Mask))
  (pad D3 smd circle (at -2.8 -2) (size 0.4 0.4) (layers F.Cu F.Paste F.Mask))
  (pad D2 smd circle (at -3.6 -2) (size 0.4 0.4) (layers F.Cu F.Paste F.Mask))
  (pad D1 smd circle (at -4.4 -2) (size 0.4 0.4) (layers F.Cu F.Paste F.Mask))
  (pad C12 smd circle (at 4.4 -2.8) (size 0.4 0.4) (layers F.Cu F.Paste F.Mask))
  (pad C11 smd circle (at 3.6 -2.8) (size 0.4 0.4) (layers F.Cu F.Paste F.Mask))
  (pad C10 smd circle (at 2.8 -2.8) (size 0.4 0.4) (layers F.Cu F.Paste F.Mask))
  (pad C9 smd circle (at 2 -2.8) (size 0.4 0.4) (layers F.Cu F.Paste F.Mask))
  (pad C8 smd circle (at 1.2 -2.8) (size 0.4 0.4) (layers F.Cu F.Paste F.Mask))
  (pad C7 smd circle (at 0.4 -2.8) (size 0.4 0.4) (layers F.Cu F.Paste F.Mask))
  (pad C6 smd circle (at -0.4 -2.8) (size 0.4 0.4) (layers F.Cu F.Paste F.Mask))
  (pad C5 smd circle (at -1.2 -2.8) (size 0.4 0.4) (layers F.Cu F.Paste F.Mask))
  (pad C4 smd circle (at -2 -2.8) (size 0.4 0.4) (layers F.Cu F.Paste F.Mask))
  (pad C3 smd circle (at -2.8 -2.8) (size 0.4 0.4) (layers F.Cu F.Paste F.Mask))
  (pad C2 smd circle (at -3.6 -2.8) (size 0.4 0.4) (layers F.Cu F.Paste F.Mask))
  (pad C1 smd circle (at -4.4 -2.8) (size 0.4 0.4) (layers F.Cu F.Paste F.Mask))
  (pad B12 smd circle (at 4.4 -3.6) (size 0.4 0.4) (layers F.Cu F.Paste F.Mask))
  (pad B11 smd circle (at 3.6 -3.6) (size 0.4 0.4) (layers F.Cu F.Paste F.Mask))
  (pad B10 smd circle (at 2.8 -3.6) (size 0.4 0.4) (layers F.Cu F.Paste F.Mask))
  (pad B9 smd circle (at 2 -3.6) (size 0.4 0.4) (layers F.Cu F.Paste F.Mask))
  (pad B8 smd circle (at 1.2 -3.6) (size 0.4 0.4) (layers F.Cu F.Paste F.Mask))
  (pad B7 smd circle (at 0.4 -3.6) (size 0.4 0.4) (layers F.Cu F.Paste F.Mask))
  (pad B6 smd circle (at -0.4 -3.6) (size 0.4 0.4) (layers F.Cu F.Paste F.Mask))
  (pad B5 smd circle (at -1.2 -3.6) (size 0.4 0.4) (layers F.Cu F.Paste F.Mask))
  (pad B4 smd circle (at -2 -3.6) (size 0.4 0.4) (layers F.Cu F.Paste F.Mask))
  (pad B3 smd circle (at -2.8 -3.6) (size 0.4 0.4) (layers F.Cu F.Paste F.Mask))
  (pad B2 smd circle (at -3.6 -3.6) (size 0.4 0.4) (layers F.Cu F.Paste F.Mask))
  (pad B1 smd circle (at -4.4 -3.6) (size 0.4 0.4) (layers F.Cu F.Paste F.Mask))
  (pad A12 smd circle (at 4.4 -4.4) (size 0.4 0.4) (layers F.Cu F.Paste F.Mask))
  (pad A11 smd circle (at 3.6 -4.4) (size 0.4 0.4) (layers F.Cu F.Paste F.Mask))
  (pad A10 smd circle (at 2.8 -4.4) (size 0.4 0.4) (layers F.Cu F.Paste F.Mask))
  (pad A9 smd circle (at 2 -4.4) (size 0.4 0.4) (layers F.Cu F.Paste F.Mask))
  (pad A8 smd circle (at 1.2 -4.4) (size 0.4 0.4) (layers F.Cu F.Paste F.Mask))
  (pad A7 smd circle (at 0.4 -4.4) (size 0.4 0.4) (layers F.Cu F.Paste F.Mask))
  (pad A6 smd circle (at -0.4 -4.4) (size 0.4 0.4) (layers F.Cu F.Paste F.Mask))
  (pad A5 smd circle (at -1.2 -4.4) (size 0.4 0.4) (layers F.Cu F.Paste F.Mask))
  (pad A4 smd circle (at -2 -4.4) (size 0.4 0.4) (layers F.Cu F.Paste F.Mask))
  (pad A3 smd circle (at -2.8 -4.4) (size 0.4 0.4) (layers F.Cu F.Paste F.Mask))
  (pad A2 smd circle (at -3.6 -4.4) (size 0.4 0.4) (layers F.Cu F.Paste F.Mask))
  (pad A1 smd circle (at -4.4 -4.4) (size 0.4 0.4) (layers F.Cu F.Paste F.Mask)))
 (gr_line (start 137.16 91.44) (end 137.16 76.2) (layer Edge.Cuts) (width 0.05))
 (gr_line (start 154.94 91.44) (end 137.16 91.44) (layer Edge.Cuts) (width 0.05))
 (gr_line (start 154.94 76.2) (end 154.94 91.44) (layer Edge.Cuts) (width 0.05))
 (gr_line (start 152.4 76.2) (end 154.94 76.2) (layer Edge.Cuts) (width 0.05))
 (gr_line (start 137.16 76.2) (end 152.4 76.2) (layer Edge.Cuts) (width 0.05))
 (segment (start 149.86 88.239) (end 151.1294 88.239) (width 0.09) (layer F.Cu) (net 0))
 (segment (start 149.86 87.439) (end 151.6258 87.439) (width 0.09) (layer F.Cu) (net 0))
 (segment (start 151.6258 87.439) (end 151.7396 87.3252) (width 0.09) (layer F.Cu) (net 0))
 (segment (start 149.86 86.639) (end 151.613 86.639) (width 0.09) (layer F.Cu) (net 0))
 (segment (start 151.613 86.639) (end 151.9428 86.3092) (width 0.09) (layer F.Cu) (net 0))
 (segment (start 149.86 85.839) (end 152.3114 85.839) (width 0.09) (layer F.Cu) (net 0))
 (segment (start 152.3238 85.8266) (end 152.3114 85.839) (width 0.09) (layer F.Cu) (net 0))
 (segment (start 149.06 85.839) (end 149.454 86.233) (width 0.09) (layer F.Cu) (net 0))
 (segment (start 149.454 86.233) (end 151.5364 86.233) (width 0.09) (layer F.Cu) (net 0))
 (segment (start 151.5364 86.233) (end 151.7142 86.0552) (width 0.09) (layer F.Cu) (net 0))
 (segment (start 151.7142 86.0552) (end 152.146 86.0552) (width 0.09) (layer F.Cu) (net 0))
 (segment (start 149.06 85.039) (end 149.4412 85.4202) (width 0.09) (layer F.Cu) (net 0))
 (segment (start 149.4412 85.4202) (end 151.4856 85.4202) (width 0.09) (layer F.Cu) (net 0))
 (segment (start 151.4856 85.4202) (end 151.511 85.3948) (width 0.09) (layer F.Cu) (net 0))
 (segment (start 149.06 84.239) (end 149.4538 84.6328) (width 0.09) (layer F.Cu) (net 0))
 (segment (start 149.4538 84.6328) (end 151.2316 84.6328) (width 0.09) (layer F.Cu) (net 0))
 (segment (start 149.86 85.039) (end 151.7648 85.039) (width 0.09) (layer F.Cu) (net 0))
 (segment (start 149.06 86.639) (end 149.4668 87.0458) (width 0.09) (layer F.Cu) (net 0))
 (segment (start 149.4668 87.0458) (end 151.6126 87.0458) (width 0.09) (layer F.Cu) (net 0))
 (segment (start 151.6126 87.0458) (end 151.6634 86.995) (width 0.09) (layer F.Cu) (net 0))
 (segment (start 148.26 85.039) (end 148.6408 85.4198) (width 0.09) (layer F.Cu) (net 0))
 (via (at 148.6408 85.4198) (size 0.45) (drill 0.2) (layers F.Cu B.Cu) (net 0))
 (segment (start 148.6408 85.4198) (end 150.9264 85.4198) (width 0.09) (layer B.Cu) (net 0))
 (segment (start 148.26 85.839) (end 148.6286 86.2076) (width 0.09) (layer F.Cu) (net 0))
 (via (at 148.6286 86.2076) (size 0.45) (drill 0.2) (layers F.Cu B.Cu) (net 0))
 (segment (start 148.6286 86.2076) (end 152.2222 86.2076) (width 0.09) (layer B.Cu) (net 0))
 (segment (start 148.26 86.639) (end 148.6414 87.0204) (width 0.09) (layer F.Cu) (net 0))
 (via (at 148.6414 87.0204) (size 0.45) (drill 0.2) (layers F.Cu B.Cu) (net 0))
 (segment (start 148.6414 87.0204) (end 151.9428 87.0204) (width 0.09) (layer B.Cu) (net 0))
 (segment (start 151.9428 87.0204) (end 152.0952 86.868) (width 0.09) (layer B.Cu) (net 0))
 (segment (start 149.5806 87.8332) (end 151.2316 87.8332) (width 0.09) (layer F.Cu) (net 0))
 (segment (start 149.1864 87.439) (end 149.5806 87.8332) (width 0.09) (layer F.Cu) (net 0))
 (segment (start 149.06 87.439) (end 149.1864 87.439) (width 0.09) (layer F.Cu) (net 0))
 (segment (start 149.4536 87.9856) (end 149.4536 88.9) (width 0.09) (layer F.Cu) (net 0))
 (segment (start 149.2878 87.8198) (end 149.4536 87.9856) (width 0.09) (layer F.Cu) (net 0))
 (segment (start 148.6408 87.8198) (end 149.2878 87.8198) (width 0.09) (layer F.Cu) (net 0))
 (segment (start 148.26 87.439) (end 148.6408 87.8198) (width 0.09) (layer F.Cu) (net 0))
 (segment (start 147.46 85.839) (end 147.8534 86.2324) (width 0.09) (layer F.Cu) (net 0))
 (via (at 147.8534 86.2324) (size 0.45) (drill 0.2) (layers F.Cu B.Cu) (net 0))
 (segment (start 147.8534 86.2324) (end 148.2604 86.6394) (width 0.09) (layer B.Cu) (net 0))
 (segment (start 148.2604 86.6394) (end 151.9682 86.6394) (width 0.09) (layer B.Cu) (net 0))
 (segment (start 151.9682 86.6394) (end 152.1206 86.487) (width 0.09) (layer B.Cu) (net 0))
 (segment (start 152.0952 86.4616) (end 152.1206 86.487) (width 0.09) (layer B.Cu) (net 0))
 (segment (start 147.46 85.039) (end 147.828 85.407) (width 0.09) (layer F.Cu) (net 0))
 (via (at 147.828 85.407) (size 0.45) (drill 0.2) (layers F.Cu B.Cu) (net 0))
 (segment (start 147.828 85.407) (end 148.2222 85.8012) (width 0.09) (layer B.Cu) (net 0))
 (segment (start 148.2222 85.8012) (end 152.0698 85.8012) (width 0.09) (layer B.Cu) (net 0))
 (segment (start 152.0698 85.8012) (end 152.2476 85.6234) (width 0.09) (layer B.Cu) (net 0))
 (segment (start 165.71 85.35) (end 164.979 85.35) (width 0.09) (layer F.Cu) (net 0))
 (segment (start 165.71 86.15) (end 165.017 86.15) (width 0.09) (layer F.Cu) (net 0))
 (segment (start 165.71 86.95) (end 165.018 86.95) (width 0.09) (layer F.Cu) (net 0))
 (segment (start 166.1095 86.5505) (end 165.1635 86.5505) (width 0.09) (layer F.Cu) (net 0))
 (segment (start 166.51 86.15) (end 166.1095 86.5505) (width 0.09) (layer F.Cu) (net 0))
 (segment (start 166.1096 85.7504) (end 165.1254 85.7504) (width 0.09) (layer F.Cu) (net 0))
 (segment (start 166.51 85.35) (end 166.1096 85.7504) (width 0.09) (layer F.Cu) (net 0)))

